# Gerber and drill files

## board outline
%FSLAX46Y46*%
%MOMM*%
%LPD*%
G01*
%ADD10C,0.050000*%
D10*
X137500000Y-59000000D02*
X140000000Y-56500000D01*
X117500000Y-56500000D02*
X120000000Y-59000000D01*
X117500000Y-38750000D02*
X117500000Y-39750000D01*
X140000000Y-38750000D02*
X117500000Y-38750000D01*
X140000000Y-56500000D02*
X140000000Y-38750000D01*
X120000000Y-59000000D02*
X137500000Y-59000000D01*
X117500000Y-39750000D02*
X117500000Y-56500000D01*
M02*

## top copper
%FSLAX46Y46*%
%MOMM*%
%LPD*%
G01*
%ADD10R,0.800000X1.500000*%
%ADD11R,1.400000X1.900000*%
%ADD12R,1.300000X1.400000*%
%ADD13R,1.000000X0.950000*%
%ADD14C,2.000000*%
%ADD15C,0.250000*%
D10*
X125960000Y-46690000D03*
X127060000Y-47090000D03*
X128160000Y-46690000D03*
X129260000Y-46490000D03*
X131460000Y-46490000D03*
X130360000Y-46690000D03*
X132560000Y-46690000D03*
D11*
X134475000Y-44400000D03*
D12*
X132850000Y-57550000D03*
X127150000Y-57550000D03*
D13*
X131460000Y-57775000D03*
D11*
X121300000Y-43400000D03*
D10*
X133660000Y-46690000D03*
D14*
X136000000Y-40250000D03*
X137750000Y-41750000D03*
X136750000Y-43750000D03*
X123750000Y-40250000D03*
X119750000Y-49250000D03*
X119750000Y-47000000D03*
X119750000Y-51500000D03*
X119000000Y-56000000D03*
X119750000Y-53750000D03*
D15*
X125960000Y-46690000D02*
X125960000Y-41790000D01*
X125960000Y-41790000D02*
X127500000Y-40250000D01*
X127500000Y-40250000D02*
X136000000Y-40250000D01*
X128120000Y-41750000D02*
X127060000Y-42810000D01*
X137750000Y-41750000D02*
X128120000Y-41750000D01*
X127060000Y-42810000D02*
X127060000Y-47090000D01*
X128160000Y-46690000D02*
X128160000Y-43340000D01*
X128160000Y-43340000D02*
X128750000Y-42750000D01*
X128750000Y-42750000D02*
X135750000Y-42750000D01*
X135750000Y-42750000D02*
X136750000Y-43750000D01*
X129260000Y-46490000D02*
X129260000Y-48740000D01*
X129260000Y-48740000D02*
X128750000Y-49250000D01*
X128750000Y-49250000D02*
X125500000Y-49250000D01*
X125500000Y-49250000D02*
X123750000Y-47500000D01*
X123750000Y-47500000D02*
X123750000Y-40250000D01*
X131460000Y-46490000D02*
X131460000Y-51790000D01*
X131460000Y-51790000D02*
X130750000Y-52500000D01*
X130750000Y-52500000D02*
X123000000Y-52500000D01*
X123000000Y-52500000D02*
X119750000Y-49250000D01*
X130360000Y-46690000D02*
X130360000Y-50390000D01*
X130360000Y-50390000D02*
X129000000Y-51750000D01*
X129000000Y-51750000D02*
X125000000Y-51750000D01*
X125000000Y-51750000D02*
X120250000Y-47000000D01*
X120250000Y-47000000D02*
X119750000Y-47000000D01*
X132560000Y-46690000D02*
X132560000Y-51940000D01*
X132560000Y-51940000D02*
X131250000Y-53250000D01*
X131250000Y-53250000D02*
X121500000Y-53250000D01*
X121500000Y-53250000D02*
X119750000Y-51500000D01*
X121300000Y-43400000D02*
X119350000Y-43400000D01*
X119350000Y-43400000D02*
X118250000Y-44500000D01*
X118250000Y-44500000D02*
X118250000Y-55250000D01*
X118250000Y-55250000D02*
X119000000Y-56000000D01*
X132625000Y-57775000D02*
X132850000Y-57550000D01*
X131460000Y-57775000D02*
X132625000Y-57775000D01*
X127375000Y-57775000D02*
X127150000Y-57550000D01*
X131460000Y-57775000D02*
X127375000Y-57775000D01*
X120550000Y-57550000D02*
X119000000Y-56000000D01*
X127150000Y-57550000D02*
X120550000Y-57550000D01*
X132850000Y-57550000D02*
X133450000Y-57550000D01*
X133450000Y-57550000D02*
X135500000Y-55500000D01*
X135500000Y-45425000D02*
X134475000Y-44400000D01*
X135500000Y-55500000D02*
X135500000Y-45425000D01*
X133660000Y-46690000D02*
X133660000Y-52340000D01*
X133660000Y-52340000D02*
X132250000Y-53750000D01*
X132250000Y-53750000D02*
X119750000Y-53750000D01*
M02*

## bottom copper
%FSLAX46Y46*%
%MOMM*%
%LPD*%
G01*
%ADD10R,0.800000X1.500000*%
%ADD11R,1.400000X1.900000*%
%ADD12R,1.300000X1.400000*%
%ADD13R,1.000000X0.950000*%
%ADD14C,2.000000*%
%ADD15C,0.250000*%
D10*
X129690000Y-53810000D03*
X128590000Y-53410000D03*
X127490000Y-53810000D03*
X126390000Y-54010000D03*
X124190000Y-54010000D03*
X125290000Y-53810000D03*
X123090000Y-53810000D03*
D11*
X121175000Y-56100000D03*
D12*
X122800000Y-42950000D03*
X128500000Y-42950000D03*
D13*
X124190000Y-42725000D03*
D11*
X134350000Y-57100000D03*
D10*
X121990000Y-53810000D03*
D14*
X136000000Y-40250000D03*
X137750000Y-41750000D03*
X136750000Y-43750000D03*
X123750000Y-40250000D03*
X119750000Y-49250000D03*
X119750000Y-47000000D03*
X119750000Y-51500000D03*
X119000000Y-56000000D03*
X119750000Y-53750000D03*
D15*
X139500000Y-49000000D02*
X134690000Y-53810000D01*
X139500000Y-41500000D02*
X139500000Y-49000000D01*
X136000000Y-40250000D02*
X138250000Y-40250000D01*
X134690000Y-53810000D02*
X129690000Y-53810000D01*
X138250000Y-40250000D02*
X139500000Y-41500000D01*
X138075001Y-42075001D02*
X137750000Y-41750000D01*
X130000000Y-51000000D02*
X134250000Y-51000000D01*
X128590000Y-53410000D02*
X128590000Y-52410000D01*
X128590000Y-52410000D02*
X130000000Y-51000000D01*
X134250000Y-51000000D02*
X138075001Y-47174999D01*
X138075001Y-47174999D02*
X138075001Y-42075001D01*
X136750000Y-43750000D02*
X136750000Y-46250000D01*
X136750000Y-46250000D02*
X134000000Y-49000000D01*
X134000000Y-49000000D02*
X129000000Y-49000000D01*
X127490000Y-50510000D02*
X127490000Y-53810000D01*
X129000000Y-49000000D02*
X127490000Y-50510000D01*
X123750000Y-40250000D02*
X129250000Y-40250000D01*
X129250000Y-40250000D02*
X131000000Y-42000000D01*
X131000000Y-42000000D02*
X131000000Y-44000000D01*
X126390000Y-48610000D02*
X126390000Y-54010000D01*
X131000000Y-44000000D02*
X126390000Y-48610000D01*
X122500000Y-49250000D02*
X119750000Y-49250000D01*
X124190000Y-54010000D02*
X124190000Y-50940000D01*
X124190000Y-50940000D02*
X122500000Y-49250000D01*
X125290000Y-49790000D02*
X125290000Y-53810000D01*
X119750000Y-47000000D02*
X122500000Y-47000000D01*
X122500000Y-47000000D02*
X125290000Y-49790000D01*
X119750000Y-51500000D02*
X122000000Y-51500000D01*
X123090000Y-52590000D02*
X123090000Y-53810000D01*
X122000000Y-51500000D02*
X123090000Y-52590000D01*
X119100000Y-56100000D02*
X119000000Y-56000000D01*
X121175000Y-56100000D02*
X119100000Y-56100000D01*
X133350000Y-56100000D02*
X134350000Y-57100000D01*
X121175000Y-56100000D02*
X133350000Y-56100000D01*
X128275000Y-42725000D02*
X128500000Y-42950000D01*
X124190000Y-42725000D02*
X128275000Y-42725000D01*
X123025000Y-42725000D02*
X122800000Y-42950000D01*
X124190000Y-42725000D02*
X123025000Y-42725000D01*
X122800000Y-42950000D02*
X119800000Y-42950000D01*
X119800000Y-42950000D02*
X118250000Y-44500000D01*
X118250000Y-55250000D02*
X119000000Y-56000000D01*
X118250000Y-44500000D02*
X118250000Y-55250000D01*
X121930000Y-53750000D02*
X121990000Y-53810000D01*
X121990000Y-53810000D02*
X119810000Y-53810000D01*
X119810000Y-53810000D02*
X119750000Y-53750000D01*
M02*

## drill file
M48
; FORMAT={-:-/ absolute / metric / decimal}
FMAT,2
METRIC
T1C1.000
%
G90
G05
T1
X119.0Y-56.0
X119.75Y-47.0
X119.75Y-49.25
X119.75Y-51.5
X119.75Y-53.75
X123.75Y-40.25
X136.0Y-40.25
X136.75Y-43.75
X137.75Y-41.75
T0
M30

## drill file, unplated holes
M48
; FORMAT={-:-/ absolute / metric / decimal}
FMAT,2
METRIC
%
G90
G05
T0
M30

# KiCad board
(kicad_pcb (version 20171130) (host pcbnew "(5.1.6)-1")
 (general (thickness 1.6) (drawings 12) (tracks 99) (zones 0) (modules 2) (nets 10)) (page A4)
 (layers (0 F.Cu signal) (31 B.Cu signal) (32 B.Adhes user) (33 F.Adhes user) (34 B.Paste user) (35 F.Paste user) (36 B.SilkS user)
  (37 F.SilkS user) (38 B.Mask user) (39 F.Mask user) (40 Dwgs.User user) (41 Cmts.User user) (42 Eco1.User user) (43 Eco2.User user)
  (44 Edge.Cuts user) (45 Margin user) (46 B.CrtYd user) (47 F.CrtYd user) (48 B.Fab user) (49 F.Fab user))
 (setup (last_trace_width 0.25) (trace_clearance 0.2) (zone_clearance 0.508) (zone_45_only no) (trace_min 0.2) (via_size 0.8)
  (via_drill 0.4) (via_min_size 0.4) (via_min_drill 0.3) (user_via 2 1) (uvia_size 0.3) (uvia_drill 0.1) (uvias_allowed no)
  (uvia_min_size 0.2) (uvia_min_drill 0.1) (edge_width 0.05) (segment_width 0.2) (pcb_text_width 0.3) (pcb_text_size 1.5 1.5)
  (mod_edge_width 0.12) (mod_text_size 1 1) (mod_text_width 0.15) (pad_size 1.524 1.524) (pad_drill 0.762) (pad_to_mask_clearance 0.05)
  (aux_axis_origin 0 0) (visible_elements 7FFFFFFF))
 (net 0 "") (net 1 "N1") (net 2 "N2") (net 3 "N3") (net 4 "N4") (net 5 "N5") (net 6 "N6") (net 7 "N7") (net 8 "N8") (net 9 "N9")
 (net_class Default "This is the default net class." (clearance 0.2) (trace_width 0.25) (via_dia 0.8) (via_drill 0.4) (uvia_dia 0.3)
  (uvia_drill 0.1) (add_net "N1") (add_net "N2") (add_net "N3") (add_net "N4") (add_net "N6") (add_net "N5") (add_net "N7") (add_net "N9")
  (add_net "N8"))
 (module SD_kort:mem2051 (layer B.Cu) (at 127.75 42.25 180)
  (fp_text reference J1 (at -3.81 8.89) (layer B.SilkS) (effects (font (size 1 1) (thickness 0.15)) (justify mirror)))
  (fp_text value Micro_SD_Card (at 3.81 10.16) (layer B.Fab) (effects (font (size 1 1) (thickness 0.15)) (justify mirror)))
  (pad 1 smd rect (at -1.94 -11.56 180) (size 0.8 1.5) (layers B.Cu B.Paste B.Mask) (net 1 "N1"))
  (pad 2 smd rect (at -0.84 -11.16 180) (size 0.8 1.5) (layers B.Cu B.Paste B.Mask) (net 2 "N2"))
  (pad 3 smd rect (at 0.26 -11.56 180) (size 0.8 1.5) (layers B.Cu B.Paste B.Mask) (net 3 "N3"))
  (pad 4 smd rect (at 1.36 -11.76 180) (size 0.8 1.5) (layers B.Cu B.Paste B.Mask) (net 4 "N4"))
  (pad 6 smd rect (at 3.56 -11.76 180) (size 0.8 1.5) (layers B.Cu B.Paste B.Mask) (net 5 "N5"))
  (pad 5 smd rect (at 2.46 -11.56 180) (size 0.8 1.5) (layers B.Cu B.Paste B.Mask) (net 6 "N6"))
  (pad 7 smd rect (at 4.66 -11.56 180) (size 0.8 1.5) (layers B.Cu B.Paste B.Mask) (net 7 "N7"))
  (pad 9 smd rect (at 6.575 -13.85 180) (size 1.4 1.9) (layers B.Cu B.Paste B.Mask) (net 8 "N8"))
  (pad 9 smd rect (at 4.95 -0.7 180) (size 1.3 1.4) (layers B.Cu B.Paste B.Mask) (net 8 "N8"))
  (pad 9 smd rect (at -0.75 -0.7 180) (size 1.3 1.4) (layers B.Cu B.Paste B.Mask) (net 8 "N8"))
  (pad 9 smd rect (at 3.56 -0.475 180) (size 1 0.95) (layers B.Cu B.Paste B.Mask) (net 8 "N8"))
  (pad 9 smd rect (at -6.6 -14.85 180) (size 1.4 1.9) (layers B.Cu B.Paste B.Mask) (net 8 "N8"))
  (pad 8 smd rect (at 5.76 -11.56 180) (size 0.8 1.5) (layers B.Cu B.Paste B.Mask) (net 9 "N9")))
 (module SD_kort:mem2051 (layer F.Cu) (at 133.5 58.25 180)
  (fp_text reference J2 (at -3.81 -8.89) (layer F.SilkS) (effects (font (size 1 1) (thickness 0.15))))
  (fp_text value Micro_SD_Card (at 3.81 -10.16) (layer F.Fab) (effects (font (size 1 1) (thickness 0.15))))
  (pad 1 smd rect (at 7.54 11.56 180) (size 0.8 1.5) (layers F.Cu F.Paste F.Mask) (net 1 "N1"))
  (pad 2 smd rect (at 6.44 11.16 180) (size 0.8 1.5) (layers F.Cu F.Paste F.Mask) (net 2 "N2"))
  (pad 3 smd rect (at 5.34 11.56 180) (size 0.8 1.5) (layers F.Cu F.Paste F.Mask) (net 3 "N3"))
  (pad 4 smd rect (at 4.24 11.76 180) (size 0.8 1.5) (layers F.Cu F.Paste F.Mask) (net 4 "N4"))
  (pad 6 smd rect (at 2.04 11.76 180) (size 0.8 1.5) (layers F.Cu F.Paste F.Mask) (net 5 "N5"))
  (pad 5 smd rect (at 3.14 11.56 180) (size 0.8 1.5) (layers F.Cu F.Paste F.Mask) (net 6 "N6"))
  (pad 7 smd rect (at 0.94 11.56 180) (size 0.8 1.5) (layers F.Cu F.Paste F.Mask) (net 7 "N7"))
  (pad 9 smd rect (at -0.975 13.85 180) (size 1.4 1.9) (layers F.Cu F.Paste F.Mask) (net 8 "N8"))
  (pad 9 smd rect (at 0.65 0.7 180) (size 1.3 1.4) (layers F.Cu F.Paste F.Mask) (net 8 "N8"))
  (pad 9 smd rect (at 6.35 0.7 180) (size 1.3 1.4) (layers F.Cu F.Paste F.Mask) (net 8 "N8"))
  (pad 9 smd rect (at 2.04 0.475 180) (size 1 0.95) (layers F.Cu F.Paste F.Mask) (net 8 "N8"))
  (pad 9 smd rect (at 12.2 14.85 180) (size 1.4 1.9) (layers F.Cu F.Paste F.Mask) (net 8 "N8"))
  (pad 8 smd rect (at -0.16 11.56 180) (size 0.8 1.5) (layers F.Cu F.Paste F.Mask) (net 9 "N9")))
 (gr_line (start 130.25 55) (end 130.25 54.25) (layer Edge.Cuts) (width 0.05))
 (gr_line (start 130 55) (end 130.25 55) (layer Edge.Cuts) (width 0.05))
 (gr_line (start 121.5 55) (end 130 55) (layer Edge.Cuts) (width 0.05))
 (gr_line (start 121.5 54.25) (end 121.5 55) (layer Edge.Cuts) (width 0.05))
 (gr_line (start 130.25 54.25) (end 121.5 54.25) (layer Edge.Cuts) (width 0.05))
 (gr_line (start 137.5 59) (end 140 56.5) (layer Edge.Cuts) (width 0.05))
 (gr_line (start 117.5 56.5) (end 120 59) (layer Edge.Cuts) (width 0.05))
 (gr_line (start 117.5 38.75) (end 117.5 39.75) (layer Edge.Cuts) (width 0.05))
 (gr_line (start 140 38.75) (end 117.5 38.75) (layer Edge.Cuts) (width 0.05))
 (gr_line (start 140 56.5) (end 140 38.75) (layer Edge.Cuts) (width 0.05))
 (gr_line (start 120 59) (end 137.5 59) (layer Edge.Cuts) (width 0.05))
 (gr_line (start 117.5 39.75) (end 117.5 56.5) (layer Edge.Cuts) (width 0.05))
 (segment (start 125.96 46.69) (end 125.96 41.79) (width 0.25) (layer F.Cu) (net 1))
 (via (at 136 40.25) (size 2) (drill 1) (layers F.Cu B.Cu) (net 1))
 (segment (start 125.96 41.79) (end 127.5 40.25) (width 0.25) (layer F.Cu) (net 1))
 (segment (start 127.5 40.25) (end 136 40.25) (width 0.25) (layer F.Cu) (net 1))
 (segment (start 139.5 49) (end 134.69 53.81) (width 0.25) (layer B.Cu) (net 1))
 (segment (start 139.5 41.5) (end 139.5 49) (width 0.25) (layer B.Cu) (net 1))
 (segment (start 136 40.25) (end 138.25 40.25) (width 0.25) (layer B.Cu) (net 1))
 (segment (start 134.69 53.81) (end 129.69 53.81) (width 0.25) (layer B.Cu) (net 1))
 (segment (start 138.25 40.25) (end 139.5 41.5) (width 0.25) (layer B.Cu) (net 1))
 (via (at 137.75 41.75) (size 2) (drill 1) (layers F.Cu B.Cu) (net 2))
 (segment (start 128.12 41.75) (end 127.06 42.81) (width 0.25) (layer F.Cu) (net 2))
 (segment (start 137.75 41.75) (end 128.12 41.75) (width 0.25) (layer F.Cu) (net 2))
 (segment (start 127.06 42.81) (end 127.06 47.09) (width 0.25) (layer F.Cu) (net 2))
 (segment (start 138.075001 42.075001) (end 137.75 41.75) (width 0.25) (layer B.Cu) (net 2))
 (segment (start 130 51) (end 134.25 51) (width 0.25) (layer B.Cu) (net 2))
 (segment (start 128.59 53.41) (end 128.59 52.41) (width 0.25) (layer B.Cu) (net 2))
 (segment (start 128.59 52.41) (end 130 51) (width 0.25) (layer B.Cu) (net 2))
 (segment (start 134.25 51) (end 138.075001 47.174999) (width 0.25) (layer B.Cu) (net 2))
 (segment (start 138.075001 47.174999) (end 138.075001 42.075001) (width 0.25) (layer B.Cu) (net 2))
 (segment (start 128.16 46.69) (end 128.16 43.34) (width 0.25) (layer F.Cu) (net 3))
 (segment (start 128.16 43.34) (end 128.75 42.75) (width 0.25) (layer F.Cu) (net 3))
 (via (at 136.75 43.75) (size 2) (drill 1) (layers F.Cu B.Cu) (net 3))
 (segment (start 128.75 42.75) (end 135.75 42.75) (width 0.25) (layer F.Cu) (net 3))
 (segment (start 135.75 42.75) (end 136.75 43.75) (width 0.25) (layer F.Cu) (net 3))
 (segment (start 136.75 43.75) (end 136.75 46.25) (width 0.25) (layer B.Cu) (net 3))
 (segment (start 136.75 46.25) (end 134 49) (width 0.25) (layer B.Cu) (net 3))
 (segment (start 134 49) (end 129 49) (width 0.25) (layer B.Cu) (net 3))
 (segment (start 127.49 50.51) (end 127.49 53.81) (width 0.25) (layer B.Cu) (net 3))
 (segment (start 129 49) (end 127.49 50.51) (width 0.25) (layer B.Cu) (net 3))
 (segment (start 129.26 46.49) (end 129.26 48.74) (width 0.25) (layer F.Cu) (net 4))
 (segment (start 129.26 48.74) (end 128.75 49.25) (width 0.25) (layer F.Cu) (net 4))
 (segment (start 128.75 49.25) (end 125.5 49.25) (width 0.25) (layer F.Cu) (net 4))
 (via (at 123.75 40.25) (size 2) (drill 1) (layers F.Cu B.Cu) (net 4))
 (segment (start 125.5 49.25) (end 123.75 47.5) (width 0.25) (layer F.Cu) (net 4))
 (segment (start 123.75 47.5) (end 123.75 40.25) (width 0.25) (layer F.Cu) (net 4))
 (segment (start 123.75 40.25) (end 129.25 40.25) (width 0.25) (layer B.Cu) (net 4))
 (segment (start 129.25 40.25) (end 131 42) (width 0.25) (layer B.Cu) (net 4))
 (segment (start 131 42) (end 131 44) (width 0.25) (layer B.Cu) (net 4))
 (segment (start 126.39 48.61) (end 126.39 54.01) (width 0.25) (layer B.Cu) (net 4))
 (segment (start 131 44) (end 126.39 48.61) (width 0.25) (layer B.Cu) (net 4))
 (segment (start 131.46 46.49) (end 131.46 51.79) (width 0.25) (layer F.Cu) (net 5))
 (segment (start 131.46 51.79) (end 130.75 52.5) (width 0.25) (layer F.Cu) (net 5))
 (via (at 119.75 49.25) (size 2) (drill 1) (layers F.Cu B.Cu) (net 5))
 (segment (start 130.75 52.5) (end 123 52.5) (width 0.25) (layer F.Cu) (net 5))
 (segment (start 123 52.5) (end 119.75 49.25) (width 0.25) (layer F.Cu) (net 5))
 (segment (start 122.5 49.25) (end 119.75 49.25) (width 0.25) (layer B.Cu) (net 5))
 (segment (start 124.19 54.01) (end 124.19 50.94) (width 0.25) (layer B.Cu) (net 5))
 (segment (start 124.19 50.94) (end 122.5 49.25) (width 0.25) (layer B.Cu) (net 5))
 (segment (start 130.36 46.69) (end 130.36 50.39) (width 0.25) (layer F.Cu) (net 6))
 (segment (start 130.36 50.39) (end 129 51.75) (width 0.25) (layer F.Cu) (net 6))
 (segment (start 129 51.75) (end 125 51.75) (width 0.25) (layer F.Cu) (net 6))
 (segment (start 125 51.75) (end 120.25 47) (width 0.25) (layer F.Cu) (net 6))
 (via (at 119.75 47) (size 2) (drill 1) (layers F.Cu B.Cu) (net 6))
 (segment (start 120.25 47) (end 119.75 47) (width 0.25) (layer F.Cu) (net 6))
 (segment (start 125.29 49.79) (end 125.29 53.81) (width 0.25) (layer B.Cu) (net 6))
 (segment (start 119.75 47) (end 122.5 47) (width 0.25) (layer B.Cu) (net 6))
 (segment (start 122.5 47) (end 125.29 49.79) (width 0.25) (layer B.Cu) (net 6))
 (segment (start 132.56 46.69) (end 132.56 51.94) (width 0.25) (layer F.Cu) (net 7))
 (segment (start 132.56 51.94) (end 131.25 53.25) (width 0.25) (layer F.Cu) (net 7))
 (via (at 119.75 51.5) (size 2) (drill 1) (layers F.Cu B.Cu) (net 7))
 (segment (start 131.25 53.25) (end 121.5 53.25) (width 0.25) (layer F.Cu) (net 7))
 (segment (start 121.5 53.25) (end 119.75 51.5) (width 0.25) (layer F.Cu) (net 7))
 (segment (start 119.75 51.5) (end 122 51.5) (width 0.25) (layer B.Cu) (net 7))
 (segment (start 123.09 52.59) (end 123.09 53.81) (width 0.25) (layer B.Cu) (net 7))
 (segment (start 122 51.5) (end 123.09 52.59) (width 0.25) (layer B.Cu) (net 7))
 (segment (start 121.3 43.4) (end 119.35 43.4) (width 0.25) (layer F.Cu) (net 8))
 (segment (start 119.35 43.4) (end 118.25 44.5) (width 0.25) (layer F.Cu) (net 8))
 (segment (start 118.25 44.5) (end 118.25 55.25) (width 0.25) (layer F.Cu) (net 8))
 (via (at 119 56) (size 2) (drill 1) (layers F.Cu B.Cu) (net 8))
 (segment (start 118.25 55.25) (end 119 56) (width 0.25) (layer F.Cu) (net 8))
 (segment (start 119.1 56.1) (end 119 56) (width 0.25) (layer B.Cu) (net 8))
 (segment (start 121.175 56.1) (end 119.1 56.1) (width 0.25) (layer B.Cu) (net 8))
 (segment (start 133.35 56.1) (end 134.35 57.1) (width 0.25) (layer B.Cu) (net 8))
 (segment (start 121.175 56.1) (end 133.35 56.1) (width 0.25) (layer B.Cu) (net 8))
 (segment (start 132.625 57.775) (end 132.85 57.55) (width 0.25) (layer F.Cu) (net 8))
 (segment (start 131.46 57.775) (end 132.625 57.775) (width 0.25) (layer F.Cu) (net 8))
 (segment (start 127.375 57.775) (end 127.15 57.55) (width 0.25) (layer F.Cu) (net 8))
 (segment (start 131.46 57.775) (end 127.375 57.775) (width 0.25) (layer F.Cu) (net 8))
 (segment (start 120.55 57.55) (end 119 56) (width 0.25) (layer F.Cu) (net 8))
 (segment (start 127.15 57.55) (end 120.55 57.55) (width 0.25) (layer F.Cu) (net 8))
 (segment (start 132.85 57.55) (end 133.45 57.55) (width 0.25) (layer F.Cu) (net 8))
 (segment (start 133.45 57.55) (end 135.5 55.5) (width 0.25) (layer F.Cu) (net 8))
 (segment (start 135.5 45.425) (end 134.475 44.4) (width 0.25) (layer F.Cu) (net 8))
 (segment (start 135.5 55.5) (end 135.5 45.425) (width 0.25) (layer F.Cu) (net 8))
 (segment (start 128.275 42.725) (end 128.5 42.95) (width 0.25) (layer B.Cu) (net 8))
 (segment (start 124.19 42.725) (end 128.275 42.725) (width 0.25) (layer B.Cu) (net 8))
 (segment (start 123.025 42.725) (end 122.8 42.95) (width 0.25) (layer B.Cu) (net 8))
 (segment (start 124.19 42.725) (end 123.025 42.725) (width 0.25) (layer B.Cu) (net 8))
 (segment (start 122.8 42.95) (end 119.8 42.95) (width 0.25) (layer B.Cu) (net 8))
 (segment (start 119.8 42.95) (end 118.25 44.5) (width 0.25) (layer B.Cu) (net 8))
 (segment (start 118.25 55.25) (end 119 56) (width 0.25) (layer B.Cu) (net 8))
 (segment (start 118.25 44.5) (end 118.25 55.25) (width 0.25) (layer B.Cu) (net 8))
 (segment (start 133.66 46.69) (end 133.66 52.34) (width 0.25) (layer F.Cu) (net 9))
 (segment (start 133.66 52.34) (end 132.25 53.75) (width 0.25) (layer F.Cu) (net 9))
 (segment (start 121.93 53.75) (end 121.99 53.81) (width 0.25) (layer B.Cu) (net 9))
 (via (at 119.75 53.75) (size 2) (drill 1) (layers F.Cu B.Cu) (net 9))
 (segment (start 121.99 53.81) (end 119.81 53.81) (width 0.25) (layer B.Cu) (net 9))
 (segment (start 119.81 53.81) (end 119.75 53.75) (width 0.25) (layer B.Cu) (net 9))
 (segment (start 132.25 53.75) (end 119.75 53.75) (width 0.25) (layer F.Cu) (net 9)))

